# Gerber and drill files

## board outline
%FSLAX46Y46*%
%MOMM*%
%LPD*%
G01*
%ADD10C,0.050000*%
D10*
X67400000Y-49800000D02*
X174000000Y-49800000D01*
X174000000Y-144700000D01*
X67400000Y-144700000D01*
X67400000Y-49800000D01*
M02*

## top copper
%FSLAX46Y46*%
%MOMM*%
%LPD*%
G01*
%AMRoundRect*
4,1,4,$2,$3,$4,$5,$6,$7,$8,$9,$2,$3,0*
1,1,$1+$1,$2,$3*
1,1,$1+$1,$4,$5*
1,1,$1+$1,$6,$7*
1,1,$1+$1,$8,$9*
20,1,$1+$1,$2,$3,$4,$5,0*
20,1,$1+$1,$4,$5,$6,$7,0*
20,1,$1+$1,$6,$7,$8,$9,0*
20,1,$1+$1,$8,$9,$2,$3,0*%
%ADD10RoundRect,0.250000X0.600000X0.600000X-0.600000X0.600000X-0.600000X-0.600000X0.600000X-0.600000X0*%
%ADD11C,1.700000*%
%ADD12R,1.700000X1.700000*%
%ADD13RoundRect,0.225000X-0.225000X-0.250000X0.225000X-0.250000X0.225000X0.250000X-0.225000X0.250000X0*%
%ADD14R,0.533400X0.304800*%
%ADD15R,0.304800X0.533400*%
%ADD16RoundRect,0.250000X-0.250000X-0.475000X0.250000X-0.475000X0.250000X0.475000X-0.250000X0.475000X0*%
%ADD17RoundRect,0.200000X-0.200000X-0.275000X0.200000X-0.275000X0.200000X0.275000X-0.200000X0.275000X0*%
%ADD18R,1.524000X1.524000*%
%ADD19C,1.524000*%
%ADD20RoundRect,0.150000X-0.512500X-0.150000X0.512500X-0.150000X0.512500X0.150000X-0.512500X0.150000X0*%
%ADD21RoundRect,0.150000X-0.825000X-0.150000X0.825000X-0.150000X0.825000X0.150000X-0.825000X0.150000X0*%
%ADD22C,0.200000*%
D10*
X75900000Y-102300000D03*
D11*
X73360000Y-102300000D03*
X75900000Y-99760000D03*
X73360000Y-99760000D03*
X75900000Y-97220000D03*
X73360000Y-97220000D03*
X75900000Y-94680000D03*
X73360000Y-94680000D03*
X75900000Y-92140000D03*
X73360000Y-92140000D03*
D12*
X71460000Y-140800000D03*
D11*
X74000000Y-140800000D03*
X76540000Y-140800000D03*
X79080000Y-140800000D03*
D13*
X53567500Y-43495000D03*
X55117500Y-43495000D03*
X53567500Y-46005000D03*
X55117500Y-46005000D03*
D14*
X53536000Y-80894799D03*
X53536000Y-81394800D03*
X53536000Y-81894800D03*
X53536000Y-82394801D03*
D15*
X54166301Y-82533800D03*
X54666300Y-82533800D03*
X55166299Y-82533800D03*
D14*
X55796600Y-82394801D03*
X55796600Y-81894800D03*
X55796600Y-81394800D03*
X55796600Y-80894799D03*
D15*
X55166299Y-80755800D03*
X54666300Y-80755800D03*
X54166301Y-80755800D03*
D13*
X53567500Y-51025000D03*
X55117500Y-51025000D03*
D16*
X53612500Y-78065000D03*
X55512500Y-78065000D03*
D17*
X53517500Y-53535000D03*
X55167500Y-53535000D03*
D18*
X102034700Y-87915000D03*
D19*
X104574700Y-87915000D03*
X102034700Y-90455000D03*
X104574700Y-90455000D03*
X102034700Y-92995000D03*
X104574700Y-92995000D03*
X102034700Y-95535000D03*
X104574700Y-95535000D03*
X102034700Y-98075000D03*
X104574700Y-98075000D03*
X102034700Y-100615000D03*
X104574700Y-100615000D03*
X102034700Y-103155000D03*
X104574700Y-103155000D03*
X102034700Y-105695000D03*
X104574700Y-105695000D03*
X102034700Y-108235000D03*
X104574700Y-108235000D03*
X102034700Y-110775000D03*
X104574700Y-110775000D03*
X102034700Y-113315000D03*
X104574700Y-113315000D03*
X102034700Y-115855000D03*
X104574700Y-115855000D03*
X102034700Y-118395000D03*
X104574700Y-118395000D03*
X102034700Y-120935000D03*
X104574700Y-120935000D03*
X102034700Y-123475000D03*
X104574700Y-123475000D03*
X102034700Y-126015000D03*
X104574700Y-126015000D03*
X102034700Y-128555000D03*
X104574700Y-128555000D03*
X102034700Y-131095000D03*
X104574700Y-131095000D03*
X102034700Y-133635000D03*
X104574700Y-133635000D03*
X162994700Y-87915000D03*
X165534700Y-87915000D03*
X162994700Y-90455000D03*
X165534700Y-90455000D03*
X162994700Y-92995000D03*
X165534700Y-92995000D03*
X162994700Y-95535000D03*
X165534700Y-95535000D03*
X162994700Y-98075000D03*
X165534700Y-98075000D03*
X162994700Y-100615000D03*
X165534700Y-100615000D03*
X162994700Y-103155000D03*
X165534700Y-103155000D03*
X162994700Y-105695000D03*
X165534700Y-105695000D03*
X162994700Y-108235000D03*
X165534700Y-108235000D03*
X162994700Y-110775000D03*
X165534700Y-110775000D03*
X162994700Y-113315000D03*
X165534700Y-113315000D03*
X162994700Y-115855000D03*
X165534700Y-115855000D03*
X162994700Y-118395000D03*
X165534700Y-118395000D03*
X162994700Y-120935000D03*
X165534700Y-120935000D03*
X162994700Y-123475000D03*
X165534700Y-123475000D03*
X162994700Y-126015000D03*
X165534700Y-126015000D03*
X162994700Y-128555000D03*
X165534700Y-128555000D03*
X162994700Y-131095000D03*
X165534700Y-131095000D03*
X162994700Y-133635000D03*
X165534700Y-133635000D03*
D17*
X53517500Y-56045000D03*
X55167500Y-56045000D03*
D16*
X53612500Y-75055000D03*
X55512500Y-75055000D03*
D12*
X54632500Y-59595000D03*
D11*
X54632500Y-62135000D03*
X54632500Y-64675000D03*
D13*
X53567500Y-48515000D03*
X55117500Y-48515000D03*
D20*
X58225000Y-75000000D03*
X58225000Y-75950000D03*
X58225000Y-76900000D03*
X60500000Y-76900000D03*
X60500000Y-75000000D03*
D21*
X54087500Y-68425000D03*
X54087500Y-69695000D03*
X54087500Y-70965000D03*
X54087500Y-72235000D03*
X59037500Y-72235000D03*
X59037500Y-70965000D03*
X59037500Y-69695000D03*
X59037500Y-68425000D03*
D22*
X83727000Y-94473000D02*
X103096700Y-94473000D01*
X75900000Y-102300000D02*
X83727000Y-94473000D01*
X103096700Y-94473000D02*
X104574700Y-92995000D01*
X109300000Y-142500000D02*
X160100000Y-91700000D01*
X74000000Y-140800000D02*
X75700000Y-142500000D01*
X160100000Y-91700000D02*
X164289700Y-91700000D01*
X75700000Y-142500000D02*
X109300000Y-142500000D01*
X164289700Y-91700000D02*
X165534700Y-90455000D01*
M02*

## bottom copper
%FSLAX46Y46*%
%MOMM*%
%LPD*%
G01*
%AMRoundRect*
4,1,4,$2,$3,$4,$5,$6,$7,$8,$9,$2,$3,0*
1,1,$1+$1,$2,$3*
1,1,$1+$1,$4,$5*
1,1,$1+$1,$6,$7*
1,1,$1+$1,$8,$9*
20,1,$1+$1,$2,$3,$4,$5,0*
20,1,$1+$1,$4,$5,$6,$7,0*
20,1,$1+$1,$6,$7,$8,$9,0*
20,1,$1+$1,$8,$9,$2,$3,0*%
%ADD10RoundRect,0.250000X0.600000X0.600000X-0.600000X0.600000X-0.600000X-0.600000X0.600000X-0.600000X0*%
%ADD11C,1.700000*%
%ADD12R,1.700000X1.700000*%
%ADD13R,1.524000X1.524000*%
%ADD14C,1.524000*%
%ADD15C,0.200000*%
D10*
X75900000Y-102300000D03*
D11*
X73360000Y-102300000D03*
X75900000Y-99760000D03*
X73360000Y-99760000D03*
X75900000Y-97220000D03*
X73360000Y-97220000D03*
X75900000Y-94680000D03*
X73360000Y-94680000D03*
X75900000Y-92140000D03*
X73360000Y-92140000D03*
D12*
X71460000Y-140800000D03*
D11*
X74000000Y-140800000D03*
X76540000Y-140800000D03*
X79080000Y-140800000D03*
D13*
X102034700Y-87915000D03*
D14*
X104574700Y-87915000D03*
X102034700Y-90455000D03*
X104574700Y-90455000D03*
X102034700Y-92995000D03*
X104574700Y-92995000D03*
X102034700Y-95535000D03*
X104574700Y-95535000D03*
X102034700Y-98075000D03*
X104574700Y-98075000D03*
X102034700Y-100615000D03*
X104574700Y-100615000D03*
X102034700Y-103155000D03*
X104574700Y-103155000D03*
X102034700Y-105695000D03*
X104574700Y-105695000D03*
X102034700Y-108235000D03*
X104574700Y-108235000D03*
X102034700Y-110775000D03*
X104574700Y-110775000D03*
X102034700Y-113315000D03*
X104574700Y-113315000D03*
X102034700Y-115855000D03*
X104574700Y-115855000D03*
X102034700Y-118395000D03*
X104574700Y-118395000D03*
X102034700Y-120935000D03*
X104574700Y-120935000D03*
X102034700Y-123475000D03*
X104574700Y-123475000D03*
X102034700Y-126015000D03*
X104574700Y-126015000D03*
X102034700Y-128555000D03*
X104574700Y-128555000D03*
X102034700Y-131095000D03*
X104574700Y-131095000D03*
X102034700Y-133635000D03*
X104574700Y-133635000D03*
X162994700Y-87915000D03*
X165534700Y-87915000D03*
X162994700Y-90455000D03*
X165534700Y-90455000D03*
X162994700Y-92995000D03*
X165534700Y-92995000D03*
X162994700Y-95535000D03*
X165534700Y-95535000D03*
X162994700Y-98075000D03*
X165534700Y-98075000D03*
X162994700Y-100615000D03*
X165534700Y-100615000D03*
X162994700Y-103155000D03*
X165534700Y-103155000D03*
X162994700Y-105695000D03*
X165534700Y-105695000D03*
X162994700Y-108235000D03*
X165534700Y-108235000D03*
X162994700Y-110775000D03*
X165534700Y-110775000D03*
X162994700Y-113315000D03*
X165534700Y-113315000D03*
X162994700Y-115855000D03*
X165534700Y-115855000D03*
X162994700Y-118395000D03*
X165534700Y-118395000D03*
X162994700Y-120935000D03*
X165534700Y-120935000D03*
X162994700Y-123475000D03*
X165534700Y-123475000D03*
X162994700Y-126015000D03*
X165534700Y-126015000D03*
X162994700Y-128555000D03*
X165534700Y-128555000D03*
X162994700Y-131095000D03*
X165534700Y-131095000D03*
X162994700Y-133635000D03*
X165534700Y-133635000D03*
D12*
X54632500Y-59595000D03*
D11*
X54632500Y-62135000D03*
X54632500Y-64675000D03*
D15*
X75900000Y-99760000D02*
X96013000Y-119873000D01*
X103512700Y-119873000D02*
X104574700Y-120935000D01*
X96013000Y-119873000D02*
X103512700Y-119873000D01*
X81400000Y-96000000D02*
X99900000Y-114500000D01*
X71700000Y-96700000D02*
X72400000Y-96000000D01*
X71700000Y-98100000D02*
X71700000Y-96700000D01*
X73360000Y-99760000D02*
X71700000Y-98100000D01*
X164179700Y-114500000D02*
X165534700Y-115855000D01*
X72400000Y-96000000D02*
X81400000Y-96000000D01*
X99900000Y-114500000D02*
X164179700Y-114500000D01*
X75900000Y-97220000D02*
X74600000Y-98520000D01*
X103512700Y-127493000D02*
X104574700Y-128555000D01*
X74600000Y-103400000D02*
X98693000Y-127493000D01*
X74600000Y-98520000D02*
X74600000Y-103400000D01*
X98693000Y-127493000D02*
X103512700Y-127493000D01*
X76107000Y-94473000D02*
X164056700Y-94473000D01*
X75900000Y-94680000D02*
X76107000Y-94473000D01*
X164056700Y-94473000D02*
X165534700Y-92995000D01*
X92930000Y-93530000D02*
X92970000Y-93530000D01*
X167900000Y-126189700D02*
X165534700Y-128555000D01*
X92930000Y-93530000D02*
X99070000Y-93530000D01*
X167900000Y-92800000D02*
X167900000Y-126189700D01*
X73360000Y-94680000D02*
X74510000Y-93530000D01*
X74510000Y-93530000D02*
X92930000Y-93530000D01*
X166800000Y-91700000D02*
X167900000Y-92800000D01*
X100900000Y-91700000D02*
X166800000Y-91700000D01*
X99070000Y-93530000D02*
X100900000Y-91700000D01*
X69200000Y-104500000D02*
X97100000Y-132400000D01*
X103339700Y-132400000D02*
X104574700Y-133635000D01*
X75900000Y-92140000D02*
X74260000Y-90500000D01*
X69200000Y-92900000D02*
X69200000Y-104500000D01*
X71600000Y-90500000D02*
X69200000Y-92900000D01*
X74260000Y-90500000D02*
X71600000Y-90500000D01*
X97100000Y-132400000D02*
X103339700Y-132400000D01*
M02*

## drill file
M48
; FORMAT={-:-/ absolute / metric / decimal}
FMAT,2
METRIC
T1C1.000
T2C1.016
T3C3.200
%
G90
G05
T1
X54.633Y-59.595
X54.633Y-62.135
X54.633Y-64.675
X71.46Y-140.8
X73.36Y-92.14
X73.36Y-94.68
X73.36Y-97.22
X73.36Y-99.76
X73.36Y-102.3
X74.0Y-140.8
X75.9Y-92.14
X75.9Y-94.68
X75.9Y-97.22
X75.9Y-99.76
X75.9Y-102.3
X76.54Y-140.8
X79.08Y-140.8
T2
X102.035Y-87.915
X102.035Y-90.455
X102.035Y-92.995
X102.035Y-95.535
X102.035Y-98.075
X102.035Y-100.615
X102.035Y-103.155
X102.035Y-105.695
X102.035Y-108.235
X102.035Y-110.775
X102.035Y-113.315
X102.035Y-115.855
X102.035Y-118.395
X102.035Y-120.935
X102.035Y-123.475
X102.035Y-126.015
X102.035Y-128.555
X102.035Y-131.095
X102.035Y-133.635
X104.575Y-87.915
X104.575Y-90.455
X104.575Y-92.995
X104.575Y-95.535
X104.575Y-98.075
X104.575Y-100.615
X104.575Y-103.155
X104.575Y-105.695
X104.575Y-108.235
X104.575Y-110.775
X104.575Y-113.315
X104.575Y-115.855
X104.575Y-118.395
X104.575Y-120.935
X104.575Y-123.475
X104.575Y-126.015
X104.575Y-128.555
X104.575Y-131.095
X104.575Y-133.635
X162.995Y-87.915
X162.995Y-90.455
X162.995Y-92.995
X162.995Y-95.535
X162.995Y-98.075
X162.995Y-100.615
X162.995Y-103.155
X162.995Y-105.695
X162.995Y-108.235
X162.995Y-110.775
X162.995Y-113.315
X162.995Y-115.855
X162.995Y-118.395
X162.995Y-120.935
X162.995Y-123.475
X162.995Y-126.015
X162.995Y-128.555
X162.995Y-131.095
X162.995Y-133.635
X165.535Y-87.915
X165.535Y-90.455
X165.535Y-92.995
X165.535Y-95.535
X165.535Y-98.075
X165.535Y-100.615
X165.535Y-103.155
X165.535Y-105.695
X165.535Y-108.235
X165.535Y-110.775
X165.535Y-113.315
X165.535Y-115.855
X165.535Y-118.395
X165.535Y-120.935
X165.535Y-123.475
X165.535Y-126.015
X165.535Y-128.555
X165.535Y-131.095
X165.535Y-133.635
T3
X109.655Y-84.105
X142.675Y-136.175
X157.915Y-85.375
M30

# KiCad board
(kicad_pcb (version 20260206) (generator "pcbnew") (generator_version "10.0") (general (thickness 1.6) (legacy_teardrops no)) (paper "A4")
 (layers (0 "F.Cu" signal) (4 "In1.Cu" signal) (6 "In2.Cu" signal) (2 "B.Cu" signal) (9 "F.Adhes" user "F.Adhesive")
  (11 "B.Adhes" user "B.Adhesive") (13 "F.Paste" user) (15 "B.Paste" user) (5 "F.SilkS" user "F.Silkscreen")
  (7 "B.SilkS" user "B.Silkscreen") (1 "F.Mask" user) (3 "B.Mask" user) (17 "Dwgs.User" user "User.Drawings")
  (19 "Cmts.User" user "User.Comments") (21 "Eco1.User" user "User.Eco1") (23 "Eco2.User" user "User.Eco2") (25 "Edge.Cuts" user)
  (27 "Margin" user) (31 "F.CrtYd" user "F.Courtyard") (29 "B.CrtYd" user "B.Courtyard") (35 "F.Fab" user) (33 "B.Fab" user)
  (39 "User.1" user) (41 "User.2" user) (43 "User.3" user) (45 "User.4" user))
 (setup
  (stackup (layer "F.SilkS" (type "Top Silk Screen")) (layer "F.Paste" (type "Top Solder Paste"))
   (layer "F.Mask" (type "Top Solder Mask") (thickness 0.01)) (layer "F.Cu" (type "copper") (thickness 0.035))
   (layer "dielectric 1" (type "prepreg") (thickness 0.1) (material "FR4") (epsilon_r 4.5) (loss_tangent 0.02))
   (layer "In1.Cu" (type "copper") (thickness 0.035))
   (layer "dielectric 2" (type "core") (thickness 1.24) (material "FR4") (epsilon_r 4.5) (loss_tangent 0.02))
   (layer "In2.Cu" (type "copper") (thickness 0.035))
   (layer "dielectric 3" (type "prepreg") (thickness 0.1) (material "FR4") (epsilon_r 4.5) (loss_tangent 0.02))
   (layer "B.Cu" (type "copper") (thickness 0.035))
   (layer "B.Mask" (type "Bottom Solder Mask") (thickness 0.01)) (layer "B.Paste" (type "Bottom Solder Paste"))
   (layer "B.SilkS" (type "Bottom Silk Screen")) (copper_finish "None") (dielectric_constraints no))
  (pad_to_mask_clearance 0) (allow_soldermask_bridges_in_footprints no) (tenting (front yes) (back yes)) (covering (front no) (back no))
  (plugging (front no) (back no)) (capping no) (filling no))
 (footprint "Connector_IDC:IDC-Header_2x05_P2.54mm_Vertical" (layer "F.Cu") (at 75.9 102.3 180)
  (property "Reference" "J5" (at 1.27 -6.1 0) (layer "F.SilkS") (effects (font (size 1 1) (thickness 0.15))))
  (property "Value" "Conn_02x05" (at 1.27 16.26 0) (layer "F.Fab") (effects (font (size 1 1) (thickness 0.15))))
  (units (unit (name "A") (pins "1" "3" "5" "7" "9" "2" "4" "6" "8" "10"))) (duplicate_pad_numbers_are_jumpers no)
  (pad "1" thru_hole roundrect (at 0 0 180) (size 1.7 1.7) (drill 1) (layers "*.Cu" "*.Mask") (remove_unused_layers no)
   (roundrect_rratio 0.147059) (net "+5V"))
  (pad "2" thru_hole circle (at 2.54 0 180) (size 1.7 1.7) (drill 1) (layers "*.Cu" "*.Mask") (remove_unused_layers no) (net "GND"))
  (pad "3" thru_hole circle (at 0 2.54 180) (size 1.7 1.7) (drill 1) (layers "*.Cu" "*.Mask") (remove_unused_layers no) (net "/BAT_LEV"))
  (pad "4" thru_hole circle (at 2.54 2.54 180) (size 1.7 1.7) (drill 1) (layers "*.Cu" "*.Mask") (remove_unused_layers no) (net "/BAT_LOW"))
  (pad "5" thru_hole circle (at 0 5.08 180) (size 1.7 1.7) (drill 1) (layers "*.Cu" "*.Mask") (remove_unused_layers no) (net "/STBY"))
  (pad "6" thru_hole circle (at 2.54 5.08 180) (size 1.7 1.7) (drill 1) (layers "*.Cu" "*.Mask") (remove_unused_layers no) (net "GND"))
  (pad "7" thru_hole circle (at 0 7.62 180) (size 1.7 1.7) (drill 1) (layers "*.Cu" "*.Mask") (remove_unused_layers no) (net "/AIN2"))
  (pad "8" thru_hole circle (at 2.54 7.62 180) (size 1.7 1.7) (drill 1) (layers "*.Cu" "*.Mask") (remove_unused_layers no) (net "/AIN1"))
  (pad "9" thru_hole circle (at 0 10.16 180) (size 1.7 1.7) (drill 1) (layers "*.Cu" "*.Mask") (remove_unused_layers no) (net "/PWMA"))
  (pad "10" thru_hole circle (at 2.54 10.16 180) (size 1.7 1.7) (drill 1) (layers "*.Cu" "*.Mask") (remove_unused_layers no) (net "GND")))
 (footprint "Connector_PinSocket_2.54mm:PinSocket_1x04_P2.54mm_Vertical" (layer "F.Cu") (at 71.46 140.8 90)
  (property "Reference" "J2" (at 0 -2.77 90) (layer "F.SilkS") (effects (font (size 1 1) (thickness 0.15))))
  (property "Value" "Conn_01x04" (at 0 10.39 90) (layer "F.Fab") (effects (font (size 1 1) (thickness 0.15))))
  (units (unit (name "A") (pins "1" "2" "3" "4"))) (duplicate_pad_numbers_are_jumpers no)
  (pad "1" thru_hole rect (at 0 0 90) (size 1.7 1.7) (drill 1) (layers "*.Cu" "*.Mask") (remove_unused_layers no) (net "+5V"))
  (pad "2" thru_hole circle (at 0 2.54 90) (size 1.7 1.7) (drill 1) (layers "*.Cu" "*.Mask") (remove_unused_layers no) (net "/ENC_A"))
  (pad "3" thru_hole circle (at 0 5.08 90) (size 1.7 1.7) (drill 1) (layers "*.Cu" "*.Mask") (remove_unused_layers no) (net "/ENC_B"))
  (pad "4" thru_hole circle (at 0 7.62 90) (size 1.7 1.7) (drill 1) (layers "*.Cu" "*.Mask") (remove_unused_layers no) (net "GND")))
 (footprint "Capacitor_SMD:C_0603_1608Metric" (layer "F.Cu") (at 54.3425 43.495)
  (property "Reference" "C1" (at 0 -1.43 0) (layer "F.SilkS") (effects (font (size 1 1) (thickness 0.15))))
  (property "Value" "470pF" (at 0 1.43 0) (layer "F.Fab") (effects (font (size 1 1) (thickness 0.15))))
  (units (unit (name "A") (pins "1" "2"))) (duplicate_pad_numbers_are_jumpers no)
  (pad "1" smd roundrect (at -0.775 0) (size 0.9 0.95) (layers "F.Cu" "F.Mask" "F.Paste") (roundrect_rratio 0.25) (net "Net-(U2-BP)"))
  (pad "2" smd roundrect (at 0.775 0) (size 0.9 0.95) (layers "F.Cu" "F.Mask" "F.Paste") (roundrect_rratio 0.25) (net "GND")))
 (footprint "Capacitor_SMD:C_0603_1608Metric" (layer "F.Cu") (at 54.3425 46.005)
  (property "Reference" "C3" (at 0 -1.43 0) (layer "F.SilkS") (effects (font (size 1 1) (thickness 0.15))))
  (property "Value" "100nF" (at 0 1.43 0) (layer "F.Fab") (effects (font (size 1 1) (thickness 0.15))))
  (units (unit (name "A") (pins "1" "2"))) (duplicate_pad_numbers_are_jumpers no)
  (pad "1" smd roundrect (at -0.775 0) (size 0.9 0.95) (layers "F.Cu" "F.Mask" "F.Paste") (roundrect_rratio 0.25) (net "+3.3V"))
  (pad "2" smd roundrect (at 0.775 0) (size 0.9 0.95) (layers "F.Cu" "F.Mask" "F.Paste") (roundrect_rratio 0.25) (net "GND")))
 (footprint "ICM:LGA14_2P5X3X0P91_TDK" (layer "F.Cu") (at 54.6663 81.6448)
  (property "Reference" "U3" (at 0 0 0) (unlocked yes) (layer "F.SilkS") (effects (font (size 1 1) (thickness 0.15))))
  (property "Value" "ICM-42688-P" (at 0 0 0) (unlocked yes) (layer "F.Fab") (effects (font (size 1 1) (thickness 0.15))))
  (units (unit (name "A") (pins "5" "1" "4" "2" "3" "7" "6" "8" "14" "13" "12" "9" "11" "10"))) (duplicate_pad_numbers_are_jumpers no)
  (pad "1" smd rect (at -1.1303 -0.750001 90) (size 0.3048 0.5334) (layers "F.Cu" "F.Mask" "F.Paste") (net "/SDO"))
  (pad "2" smd rect (at -1.1303 -0.25 90) (size 0.3048 0.5334) (layers "F.Cu" "F.Mask" "F.Paste") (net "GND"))
  (pad "3" smd rect (at -1.1303 0.25 90) (size 0.3048 0.5334) (layers "F.Cu" "F.Mask" "F.Paste") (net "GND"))
  (pad "4" smd rect (at -1.1303 0.750001 90) (size 0.3048 0.5334) (layers "F.Cu" "F.Mask" "F.Paste") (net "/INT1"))
  (pad "5" smd rect (at -0.499999 0.889) (size 0.3048 0.5334) (layers "F.Cu" "F.Mask" "F.Paste") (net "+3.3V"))
  (pad "6" smd rect (at 0 0.889) (size 0.3048 0.5334) (layers "F.Cu" "F.Mask" "F.Paste") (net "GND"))
  (pad "7" smd rect (at 0.499999 0.889) (size 0.3048 0.5334) (layers "F.Cu" "F.Mask" "F.Paste") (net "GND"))
  (pad "8" smd rect (at 1.1303 0.750001 90) (size 0.3048 0.5334) (layers "F.Cu" "F.Mask" "F.Paste") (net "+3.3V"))
  (pad "9" smd rect (at 1.1303 0.25 90) (size 0.3048 0.5334) (layers "F.Cu" "F.Mask" "F.Paste") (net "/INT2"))
  (pad "10" smd rect (at 1.1303 -0.25 90) (size 0.3048 0.5334) (layers "F.Cu" "F.Mask" "F.Paste") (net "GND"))
  (pad "11" smd rect (at 1.1303 -0.750001 90) (size 0.3048 0.5334) (layers "F.Cu" "F.Mask" "F.Paste") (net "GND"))
  (pad "12" smd rect (at 0.499999 -0.889) (size 0.3048 0.5334) (layers "F.Cu" "F.Mask" "F.Paste") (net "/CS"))
  (pad "13" smd rect (at 0 -0.889) (size 0.3048 0.5334) (layers "F.Cu" "F.Mask" "F.Paste") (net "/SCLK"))
  (pad "14" smd rect (at -0.499999 -0.889) (size 0.3048 0.5334) (layers "F.Cu" "F.Mask" "F.Paste") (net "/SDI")))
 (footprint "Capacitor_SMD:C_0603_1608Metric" (layer "F.Cu") (at 54.3425 51.025)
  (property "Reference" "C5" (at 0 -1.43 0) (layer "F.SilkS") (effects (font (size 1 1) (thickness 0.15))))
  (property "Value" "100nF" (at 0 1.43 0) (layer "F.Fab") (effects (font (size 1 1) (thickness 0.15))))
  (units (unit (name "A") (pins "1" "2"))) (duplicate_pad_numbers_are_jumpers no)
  (pad "1" smd roundrect (at -0.775 0) (size 0.9 0.95) (layers "F.Cu" "F.Mask" "F.Paste") (roundrect_rratio 0.25) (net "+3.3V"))
  (pad "2" smd roundrect (at 0.775 0) (size 0.9 0.95) (layers "F.Cu" "F.Mask" "F.Paste") (roundrect_rratio 0.25) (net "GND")))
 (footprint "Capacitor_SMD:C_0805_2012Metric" (layer "F.Cu") (at 54.5625 78.065)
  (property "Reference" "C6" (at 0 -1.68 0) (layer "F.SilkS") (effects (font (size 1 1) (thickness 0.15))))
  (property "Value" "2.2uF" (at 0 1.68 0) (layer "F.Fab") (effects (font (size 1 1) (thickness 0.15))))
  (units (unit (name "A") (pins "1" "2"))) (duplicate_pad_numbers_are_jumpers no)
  (pad "1" smd roundrect (at -0.95 0) (size 1 1.45) (layers "F.Cu" "F.Mask" "F.Paste") (roundrect_rratio 0.25) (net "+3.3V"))
  (pad "2" smd roundrect (at 0.95 0) (size 1 1.45) (layers "F.Cu" "F.Mask" "F.Paste") (roundrect_rratio 0.25) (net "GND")))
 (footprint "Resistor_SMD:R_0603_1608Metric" (layer "F.Cu") (at 54.3425 53.535)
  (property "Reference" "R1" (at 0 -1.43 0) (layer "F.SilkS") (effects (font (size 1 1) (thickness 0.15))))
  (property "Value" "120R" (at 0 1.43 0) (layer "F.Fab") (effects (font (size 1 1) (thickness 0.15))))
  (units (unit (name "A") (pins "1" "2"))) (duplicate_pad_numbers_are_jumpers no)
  (pad "1" smd roundrect (at -0.825 0) (size 0.8 0.95) (layers "F.Cu" "F.Mask" "F.Paste") (roundrect_rratio 0.25) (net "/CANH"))
  (pad "2" smd roundrect (at 0.825 0) (size 0.8 0.95) (layers "F.Cu" "F.Mask" "F.Paste") (roundrect_rratio 0.25) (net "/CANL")))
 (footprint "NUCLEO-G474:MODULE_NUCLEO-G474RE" (layer "F.Cu") (at 133.7847 97.425)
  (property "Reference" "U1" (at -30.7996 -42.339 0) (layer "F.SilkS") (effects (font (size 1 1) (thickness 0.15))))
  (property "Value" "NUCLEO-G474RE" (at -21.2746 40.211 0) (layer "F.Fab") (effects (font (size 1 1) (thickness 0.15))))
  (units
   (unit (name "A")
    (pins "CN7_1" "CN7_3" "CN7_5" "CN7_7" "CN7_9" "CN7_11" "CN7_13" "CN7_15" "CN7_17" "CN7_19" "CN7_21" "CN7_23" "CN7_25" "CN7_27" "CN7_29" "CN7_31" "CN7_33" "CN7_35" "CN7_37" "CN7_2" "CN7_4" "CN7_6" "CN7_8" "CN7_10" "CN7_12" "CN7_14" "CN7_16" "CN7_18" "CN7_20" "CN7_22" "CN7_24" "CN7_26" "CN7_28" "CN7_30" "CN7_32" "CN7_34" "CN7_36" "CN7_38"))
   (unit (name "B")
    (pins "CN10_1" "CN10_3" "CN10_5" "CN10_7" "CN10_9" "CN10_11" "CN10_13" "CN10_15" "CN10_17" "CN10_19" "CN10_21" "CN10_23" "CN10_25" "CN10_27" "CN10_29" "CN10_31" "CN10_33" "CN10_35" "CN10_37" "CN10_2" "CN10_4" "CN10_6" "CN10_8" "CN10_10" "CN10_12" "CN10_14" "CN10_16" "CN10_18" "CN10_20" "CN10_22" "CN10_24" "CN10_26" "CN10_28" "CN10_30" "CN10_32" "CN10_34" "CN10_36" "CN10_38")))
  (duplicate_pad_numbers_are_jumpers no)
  (pad "" np_thru_hole circle (at -24.13 -13.32) (size 3.2 3.2) (drill 3.2) (layers "*.Cu" "*.Mask"))
  (pad "" np_thru_hole circle (at 8.89 38.75) (size 3.2 3.2) (drill 3.2) (layers "*.Cu" "*.Mask"))
  (pad "" np_thru_hole circle (at 24.13 -12.05) (size 3.2 3.2) (drill 3.2) (layers "*.Cu" "*.Mask"))
  (pad "CN7_1" thru_hole rect (at -31.75 -9.51) (size 1.524 1.524) (drill 1.016) (layers "*.Cu" "*.Mask") (remove_unused_layers no)
   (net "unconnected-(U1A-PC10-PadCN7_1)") (solder_mask_margin 0.102))
  (pad "CN7_2" thru_hole circle (at -29.21 -9.51) (size 1.524 1.524) (drill 1.016) (layers "*.Cu" "*.Mask") (remove_unused_layers no)
   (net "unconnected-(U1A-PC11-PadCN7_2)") (solder_mask_margin 0.102))
  (pad "CN7_3" thru_hole circle (at -31.75 -6.97) (size 1.524 1.524) (drill 1.016) (layers "*.Cu" "*.Mask") (remove_unused_layers no)
   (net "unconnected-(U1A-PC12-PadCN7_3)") (solder_mask_margin 0.102))
  (pad "CN7_4" thru_hole circle (at -29.21 -6.97) (size 1.524 1.524) (drill 1.016) (layers "*.Cu" "*.Mask") (remove_unused_layers no)
   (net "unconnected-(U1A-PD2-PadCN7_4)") (solder_mask_margin 0.102))
  (pad "CN7_5" thru_hole circle (at -31.75 -4.43) (size 1.524 1.524) (drill 1.016) (layers "*.Cu" "*.Mask") (remove_unused_layers no)
   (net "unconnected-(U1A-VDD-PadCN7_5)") (solder_mask_margin 0.102))
  (pad "CN7_6" thru_hole circle (at -29.21 -4.43) (size 1.524 1.524) (drill 1.016) (layers "*.Cu" "*.Mask") (remove_unused_layers no)
   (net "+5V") (solder_mask_margin 0.102))
  (pad "CN7_7" thru_hole circle (at -31.75 -1.89) (size 1.524 1.524) (drill 1.016) (layers "*.Cu" "*.Mask") (remove_unused_layers no)
   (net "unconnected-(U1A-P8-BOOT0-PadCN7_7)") (solder_mask_margin 0.102))
  (pad "CN7_8" thru_hole circle (at -29.21 -1.89) (size 1.524 1.524) (drill 1.016) (layers "*.Cu" "*.Mask") (remove_unused_layers no)
   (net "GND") (solder_mask_margin 0.102))
  (pad "CN7_9" thru_hole circle (at -31.75 0.65) (size 1.524 1.524) (drill 1.016) (layers "*.Cu" "*.Mask") (remove_unused_layers no)
   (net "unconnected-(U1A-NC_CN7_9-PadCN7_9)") (solder_mask_margin 0.102))
  (pad "CN7_10" thru_hole circle (at -29.21 0.65) (size 1.524 1.524) (drill 1.016) (layers "*.Cu" "*.Mask") (remove_unused_layers no)
   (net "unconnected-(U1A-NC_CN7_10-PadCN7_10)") (solder_mask_margin 0.102))
  (pad "CN7_11" thru_hole circle (at -31.75 3.19) (size 1.524 1.524) (drill 1.016) (layers "*.Cu" "*.Mask") (remove_unused_layers no)
   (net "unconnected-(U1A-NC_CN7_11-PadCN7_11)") (solder_mask_margin 0.102))
  (pad "CN7_12" thru_hole circle (at -29.21 3.19) (size 1.524 1.524) (drill 1.016) (layers "*.Cu" "*.Mask") (remove_unused_layers no)
   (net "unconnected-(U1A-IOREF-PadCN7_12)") (solder_mask_margin 0.102))
  (pad "CN7_13" thru_hole circle (at -31.75 5.73) (size 1.524 1.524) (drill 1.016) (layers "*.Cu" "*.Mask") (remove_unused_layers no)
   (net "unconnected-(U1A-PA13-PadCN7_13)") (solder_mask_margin 0.102))
  (pad "CN7_14" thru_hole circle (at -29.21 5.73) (size 1.524 1.524) (drill 1.016) (layers "*.Cu" "*.Mask") (remove_unused_layers no)
   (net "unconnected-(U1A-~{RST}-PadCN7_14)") (solder_mask_margin 0.102))
  (pad "CN7_15" thru_hole circle (at -31.75 8.27) (size 1.524 1.524) (drill 1.016) (layers "*.Cu" "*.Mask") (remove_unused_layers no)
   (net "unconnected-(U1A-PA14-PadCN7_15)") (solder_mask_margin 0.102))
  (pad "CN7_16" thru_hole circle (at -29.21 8.27) (size 1.524 1.524) (drill 1.016) (layers "*.Cu" "*.Mask") (remove_unused_layers no)
   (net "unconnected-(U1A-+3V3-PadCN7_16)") (solder_mask_margin 0.102))
  (pad "CN7_17" thru_hole circle (at -31.75 10.81) (size 1.524 1.524) (drill 1.016) (layers "*.Cu" "*.Mask") (remove_unused_layers no)
   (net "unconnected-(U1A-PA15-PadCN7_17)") (solder_mask_margin 0.102))
  (pad "CN7_18" thru_hole circle (at -29.21 10.81) (size 1.524 1.524) (drill 1.016) (layers "*.Cu" "*.Mask") (remove_unused_layers no)
   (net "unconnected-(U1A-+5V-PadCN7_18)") (solder_mask_margin 0.102))
  (pad "CN7_19" thru_hole circle (at -31.75 13.35) (size 1.524 1.524) (drill 1.016) (layers "*.Cu" "*.Mask") (remove_unused_layers no)
   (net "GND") (solder_mask_margin 0.102))
  (pad "CN7_20" thru_hole circle (at -29.21 13.35) (size 1.524 1.524) (drill 1.016) (layers "*.Cu" "*.Mask") (remove_unused_layers no)
   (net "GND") (solder_mask_margin 0.102))
  (pad "CN7_21" thru_hole circle (at -31.75 15.89) (size 1.524 1.524) (drill 1.016) (layers "*.Cu" "*.Mask") (remove_unused_layers no)
   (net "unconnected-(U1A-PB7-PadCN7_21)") (solder_mask_margin 0.102))
  (pad "CN7_22" thru_hole circle (at -29.21 15.89) (size 1.524 1.524) (drill 1.016) (layers "*.Cu" "*.Mask") (remove_unused_layers no)
   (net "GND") (solder_mask_margin 0.102))
  (pad "CN7_23" thru_hole circle (at -31.75 18.43) (size 1.524 1.524) (drill 1.016) (layers "*.Cu" "*.Mask") (remove_unused_layers no)
   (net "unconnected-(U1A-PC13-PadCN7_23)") (solder_mask_margin 0.102))
  (pad "CN7_24" thru_hole circle (at -29.21 18.43) (size 1.524 1.524) (drill 1.016) (layers "*.Cu" "*.Mask") (remove_unused_layers no)
   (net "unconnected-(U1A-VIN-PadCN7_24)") (solder_mask_margin 0.102))
  (pad "CN7_25" thru_hole circle (at -31.75 20.97) (size 1.524 1.524) (drill 1.016) (layers "*.Cu" "*.Mask") (remove_unused_layers no)
   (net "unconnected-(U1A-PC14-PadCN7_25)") (solder_mask_margin 0.102))
  (pad "CN7_26" thru_hole circle (at -29.21 20.97) (size 1.524 1.524) (drill 1.016) (layers "*.Cu" "*.Mask") (remove_unused_layers no)
   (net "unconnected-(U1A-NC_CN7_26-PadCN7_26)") (solder_mask_margin 0.102))
  (pad "CN7_27" thru_hole circle (at -31.75 23.51) (size 1.524 1.524) (drill 1.016) (layers "*.Cu" "*.Mask") (remove_unused_layers no)
   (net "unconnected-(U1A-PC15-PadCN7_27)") (solder_mask_margin 0.102))
  (pad "CN7_28" thru_hole circle (at -29.21 23.51) (size 1.524 1.524) (drill 1.016) (layers "*.Cu" "*.Mask") (remove_unused_layers no)
   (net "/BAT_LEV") (solder_mask_margin 0.102))
  (pad "CN7_29" thru_hole circle (at -31.75 26.05) (size 1.524 1.524) (drill 1.016) (layers "*.Cu" "*.Mask") (remove_unused_layers no)
   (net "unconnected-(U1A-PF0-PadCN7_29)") (solder_mask_margin 0.102))
  (pad "CN7_30" thru_hole circle (at -29.21 26.05) (size 1.524 1.524) (drill 1.016) (layers "*.Cu" "*.Mask") (remove_unused_layers no)
   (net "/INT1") (solder_mask_margin 0.102))
  (pad "CN7_31" thru_hole circle (at -31.75 28.59) (size 1.524 1.524) (drill 1.016) (layers "*.Cu" "*.Mask") (remove_unused_layers no)
   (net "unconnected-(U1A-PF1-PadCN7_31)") (solder_mask_margin 0.102))
  (pad "CN7_32" thru_hole circle (at -29.21 28.59) (size 1.524 1.524) (drill 1.016) (layers "*.Cu" "*.Mask") (remove_unused_layers no)
   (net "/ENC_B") (solder_mask_margin 0.102))
  (pad "CN7_33" thru_hole circle (at -31.75 31.13) (size 1.524 1.524) (drill 1.016) (layers "*.Cu" "*.Mask") (remove_unused_layers no)
   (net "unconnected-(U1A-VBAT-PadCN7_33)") (solder_mask_margin 0.102))
  (pad "CN7_34" thru_hole circle (at -29.21 31.13) (size 1.524 1.524) (drill 1.016) (layers "*.Cu" "*.Mask") (remove_unused_layers no)
   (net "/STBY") (solder_mask_margin 0.102))
  (pad "CN7_35" thru_hole circle (at -31.75 33.67) (size 1.524 1.524) (drill 1.016) (layers "*.Cu" "*.Mask") (remove_unused_layers no)
   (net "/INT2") (solder_mask_margin 0.102))
  (pad "CN7_36" thru_hole circle (at -29.21 33.67) (size 1.524 1.524) (drill 1.016) (layers "*.Cu" "*.Mask") (remove_unused_layers no)
   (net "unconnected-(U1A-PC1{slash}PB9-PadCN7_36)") (solder_mask_margin 0.102))
  (pad "CN7_37" thru_hole circle (at -31.75 36.21) (size 1.524 1.524) (drill 1.016) (layers "*.Cu" "*.Mask") (remove_unused_layers no)
   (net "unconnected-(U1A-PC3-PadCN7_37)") (solder_mask_margin 0.102))
  (pad "CN7_38" thru_hole circle (at -29.21 36.21) (size 1.524 1.524) (drill 1.016) (layers "*.Cu" "*.Mask") (remove_unused_layers no)
   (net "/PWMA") (solder_mask_margin 0.102))
  (pad "CN10_1" thru_hole circle (at 29.21 -9.51) (size 1.524 1.524) (drill 1.016) (layers "*.Cu" "*.Mask") (remove_unused_layers no)
   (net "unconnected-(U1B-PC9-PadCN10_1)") (solder_mask_margin 0.102))
  (pad "CN10_2" thru_hole circle (at 31.75 -9.51) (size 1.524 1.524) (drill 1.016) (layers "*.Cu" "*.Mask") (remove_unused_layers no)
   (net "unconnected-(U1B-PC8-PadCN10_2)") (solder_mask_margin 0.102))
  (pad "CN10_3" thru_hole circle (at 29.21 -6.97) (size 1.524 1.524) (drill 1.016) (layers "*.Cu" "*.Mask") (remove_unused_layers no)
   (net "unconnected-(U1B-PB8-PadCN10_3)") (solder_mask_margin 0.102))
  (pad "CN10_4" thru_hole circle (at 31.75 -6.97) (size 1.524 1.524) (drill 1.016) (layers "*.Cu" "*.Mask") (remove_unused_layers no)
   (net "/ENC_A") (solder_mask_margin 0.102))
  (pad "CN10_5" thru_hole circle (at 29.21 -4.43) (size 1.524 1.524) (drill 1.016) (layers "*.Cu" "*.Mask") (remove_unused_layers no)
   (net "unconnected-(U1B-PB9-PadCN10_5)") (solder_mask_margin 0.102))
  (pad "CN10_6" thru_hole circle (at 31.75 -4.43) (size 1.524 1.524) (drill 1.016) (layers "*.Cu" "*.Mask") (remove_unused_layers no)
   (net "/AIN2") (solder_mask_margin 0.102))
  (pad "CN10_7" thru_hole circle (at 29.21 -1.89) (size 1.524 1.524) (drill 1.016) (layers "*.Cu" "*.Mask") (remove_unused_layers no)
   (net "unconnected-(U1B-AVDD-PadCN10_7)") (solder_mask_margin 0.102))
  (pad "CN10_8" thru_hole circle (at 31.75 -1.89) (size 1.524 1.524) (drill 1.016) (layers "*.Cu" "*.Mask") (remove_unused_layers no)
   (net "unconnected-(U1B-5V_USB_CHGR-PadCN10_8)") (solder_mask_margin 0.102))
  (pad "CN10_9" thru_hole circle (at 29.21 0.65) (size 1.524 1.524) (drill 1.016) (layers "*.Cu" "*.Mask") (remove_unused_layers no)
   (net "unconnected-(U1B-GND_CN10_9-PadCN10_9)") (solder_mask_margin 0.102))
  (pad "CN10_10" thru_hole circle (at 31.75 0.65) (size 1.524 1.524) (drill 1.016) (layers "*.Cu" "*.Mask") (remove_unused_layers no)
   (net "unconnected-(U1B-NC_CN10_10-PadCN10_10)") (solder_mask_margin 0.102))
  (pad "CN10_11" thru_hole circle (at 29.21 3.19) (size 1.524 1.524) (drill 1.016) (layers "*.Cu" "*.Mask") (remove_unused_layers no)
   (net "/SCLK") (solder_mask_margin 0.102))
  (pad "CN10_12" thru_hole circle (at 31.75 3.19) (size 1.524 1.524) (drill 1.016) (layers "*.Cu" "*.Mask") (remove_unused_layers no)
   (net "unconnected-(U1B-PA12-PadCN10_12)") (solder_mask_margin 0.102))
  (pad "CN10_13" thru_hole circle (at 29.21 5.73) (size 1.524 1.524) (drill 1.016) (layers "*.Cu" "*.Mask") (remove_unused_layers no)
   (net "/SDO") (solder_mask_margin 0.102))
  (pad "CN10_14" thru_hole circle (at 31.75 5.73) (size 1.524 1.524) (drill 1.016) (layers "*.Cu" "*.Mask") (remove_unused_layers no)
   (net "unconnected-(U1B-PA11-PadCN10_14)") (solder_mask_margin 0.102))
  (pad "CN10_15" thru_hole circle (at 29.21 8.27) (size 1.524 1.524) (drill 1.016) (layers "*.Cu" "*.Mask") (remove_unused_layers no)
   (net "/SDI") (solder_mask_margin 0.102))
  (pad "CN10_16" thru_hole circle (at 31.75 8.27) (size 1.524 1.524) (drill 1.016) (layers "*.Cu" "*.Mask") (remove_unused_layers no)
   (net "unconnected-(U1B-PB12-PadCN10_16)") (solder_mask_margin 0.102))
  (pad "CN10_17" thru_hole circle (at 29.21 10.81) (size 1.524 1.524) (drill 1.016) (layers "*.Cu" "*.Mask") (remove_unused_layers no)
   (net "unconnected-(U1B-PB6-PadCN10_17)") (solder_mask_margin 0.102))
  (pad "CN10_18" thru_hole circle (at 31.75 10.81) (size 1.524 1.524) (drill 1.016) (layers "*.Cu" "*.Mask") (remove_unused_layers no)
   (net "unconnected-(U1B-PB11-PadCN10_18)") (solder_mask_margin 0.102))
  (pad "CN10_19" thru_hole circle (at 29.21 13.35) (size 1.524 1.524) (drill 1.016) (layers "*.Cu" "*.Mask") (remove_unused_layers no)
   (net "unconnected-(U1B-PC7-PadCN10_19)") (solder_mask_margin 0.102))
  (pad "CN10_20" thru_hole circle (at 31.75 13.35) (size 1.524 1.524) (drill 1.016) (layers "*.Cu" "*.Mask") (remove_unused_layers no)
   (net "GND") (solder_mask_margin 0.102))
  (pad "CN10_21" thru_hole circle (at 29.21 15.89) (size 1.524 1.524) (drill 1.016) (layers "*.Cu" "*.Mask") (remove_unused_layers no)
   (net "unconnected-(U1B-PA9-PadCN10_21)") (solder_mask_margin 0.102))
  (pad "CN10_22" thru_hole circle (at 31.75 15.89) (size 1.524 1.524) (drill 1.016) (layers "*.Cu" "*.Mask") (remove_unused_layers no)
   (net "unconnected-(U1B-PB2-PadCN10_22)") (solder_mask_margin 0.102))
  (pad "CN10_23" thru_hole circle (at 29.21 18.43) (size 1.524 1.524) (drill 1.016) (layers "*.Cu" "*.Mask") (remove_unused_layers no)
   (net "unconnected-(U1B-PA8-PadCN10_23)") (solder_mask_margin 0.102))
  (pad "CN10_24" thru_hole circle (at 31.75 18.43) (size 1.524 1.524) (drill 1.016) (layers "*.Cu" "*.Mask") (remove_unused_layers no)
   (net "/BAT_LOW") (solder_mask_margin 0.102))
  (pad "CN10_25" thru_hole circle (at 29.21 20.97) (size 1.524 1.524) (drill 1.016) (layers "*.Cu" "*.Mask") (remove_unused_layers no)
   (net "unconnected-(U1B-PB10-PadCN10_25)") (solder_mask_margin 0.102))
  (pad "CN10_26" thru_hole circle (at 31.75 20.97) (size 1.524 1.524) (drill 1.016) (layers "*.Cu" "*.Mask") (remove_unused_layers no)
   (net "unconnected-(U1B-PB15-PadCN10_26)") (solder_mask_margin 0.102))
  (pad "CN10_27" thru_hole circle (at 29.21 23.51) (size 1.524 1.524) (drill 1.016) (layers "*.Cu" "*.Mask") (remove_unused_layers no)
   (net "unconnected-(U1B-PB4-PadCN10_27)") (solder_mask_margin 0.102))
  (pad "CN10_28" thru_hole circle (at 31.75 23.51) (size 1.524 1.524) (drill 1.016) (layers "*.Cu" "*.Mask") (remove_unused_layers no)
   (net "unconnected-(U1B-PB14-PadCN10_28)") (solder_mask_margin 0.102))
  (pad "CN10_29" thru_hole circle (at 29.21 26.05) (size 1.524 1.524) (drill 1.016) (layers "*.Cu" "*.Mask") (remove_unused_layers no)
   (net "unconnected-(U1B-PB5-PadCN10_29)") (solder_mask_margin 0.102))
  (pad "CN10_30" thru_hole circle (at 31.75 26.05) (size 1.524 1.524) (drill 1.016) (layers "*.Cu" "*.Mask") (remove_unused_layers no)
   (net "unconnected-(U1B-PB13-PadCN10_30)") (solder_mask_margin 0.102))
  (pad "CN10_31" thru_hole circle (at 29.21 28.59) (size 1.524 1.524) (drill 1.016) (layers "*.Cu" "*.Mask") (remove_unused_layers no)
   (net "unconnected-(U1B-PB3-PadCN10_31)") (solder_mask_margin 0.102))
  (pad "CN10_32" thru_hole circle (at 31.75 28.59) (size 1.524 1.524) (drill 1.016) (layers "*.Cu" "*.Mask") (remove_unused_layers no)
   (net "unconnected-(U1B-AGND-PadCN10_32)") (solder_mask_margin 0.102))
  (pad "CN10_33" thru_hole circle (at 29.21 31.13) (size 1.524 1.524) (drill 1.016) (layers "*.Cu" "*.Mask") (remove_unused_layers no)
   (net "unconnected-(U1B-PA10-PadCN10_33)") (solder_mask_margin 0.102))
  (pad "CN10_34" thru_hole circle (at 31.75 31.13) (size 1.524 1.524) (drill 1.016) (layers "*.Cu" "*.Mask") (remove_unused_layers no)
   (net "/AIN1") (solder_mask_margin 0.102))
  (pad "CN10_35" thru_hole circle (at 29.21 33.67) (size 1.524 1.524) (drill 1.016) (layers "*.Cu" "*.Mask") (remove_unused_layers no)
   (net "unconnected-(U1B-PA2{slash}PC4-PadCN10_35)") (solder_mask_margin 0.102))
  (pad "CN10_36" thru_hole circle (at 31.75 33.67) (size 1.524 1.524) (drill 1.016) (layers "*.Cu" "*.Mask") (remove_unused_layers no)
   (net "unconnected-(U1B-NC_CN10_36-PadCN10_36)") (solder_mask_margin 0.102))
  (pad "CN10_37" thru_hole circle (at 29.21 36.21) (size 1.524 1.524) (drill 1.016) (layers "*.Cu" "*.Mask") (remove_unused_layers no)
   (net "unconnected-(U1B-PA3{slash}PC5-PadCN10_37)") (solder_mask_margin 0.102))
  (pad "CN10_38" thru_hole circle (at 31.75 36.21) (size 1.524 1.524) (drill 1.016) (layers "*.Cu" "*.Mask") (remove_unused_layers no)
   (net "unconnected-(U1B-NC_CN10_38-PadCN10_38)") (solder_mask_margin 0.102)))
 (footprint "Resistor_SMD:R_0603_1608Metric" (layer "F.Cu") (at 54.3425 56.045)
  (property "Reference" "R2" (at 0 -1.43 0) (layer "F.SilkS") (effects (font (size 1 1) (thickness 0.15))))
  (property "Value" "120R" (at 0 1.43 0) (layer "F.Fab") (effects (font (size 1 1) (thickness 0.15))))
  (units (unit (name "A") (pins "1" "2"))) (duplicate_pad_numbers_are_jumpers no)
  (pad "1" smd roundrect (at -0.825 0) (size 0.8 0.95) (layers "F.Cu" "F.Mask" "F.Paste") (roundrect_rratio 0.25) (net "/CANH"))
  (pad "2" smd roundrect (at 0.825 0) (size 0.8 0.95) (layers "F.Cu" "F.Mask" "F.Paste") (roundrect_rratio 0.25) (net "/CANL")))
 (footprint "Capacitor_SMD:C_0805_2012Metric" (layer "F.Cu") (at 54.5625 75.055)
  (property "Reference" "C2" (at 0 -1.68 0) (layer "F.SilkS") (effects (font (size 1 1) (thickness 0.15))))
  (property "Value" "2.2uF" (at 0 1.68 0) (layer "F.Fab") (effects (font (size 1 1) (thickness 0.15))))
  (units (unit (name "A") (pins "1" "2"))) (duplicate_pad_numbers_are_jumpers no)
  (pad "1" smd roundrect (at -0.95 0) (size 1 1.45) (layers "F.Cu" "F.Mask" "F.Paste") (roundrect_rratio 0.25) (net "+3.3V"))
  (pad "2" smd roundrect (at 0.95 0) (size 1 1.45) (layers "F.Cu" "F.Mask" "F.Paste") (roundrect_rratio 0.25) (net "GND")))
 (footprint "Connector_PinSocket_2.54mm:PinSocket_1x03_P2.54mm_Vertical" (layer "F.Cu") (at 54.6325 59.595)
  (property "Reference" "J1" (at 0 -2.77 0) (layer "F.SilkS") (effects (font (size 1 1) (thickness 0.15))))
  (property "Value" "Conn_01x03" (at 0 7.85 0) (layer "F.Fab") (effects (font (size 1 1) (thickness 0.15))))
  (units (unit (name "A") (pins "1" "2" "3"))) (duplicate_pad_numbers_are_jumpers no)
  (pad "1" thru_hole rect (at 0 0) (size 1.7 1.7) (drill 1) (layers "*.Cu" "*.Mask") (remove_unused_layers no) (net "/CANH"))
  (pad "2" thru_hole circle (at 0 2.54) (size 1.7 1.7) (drill 1) (layers "*.Cu" "*.Mask") (remove_unused_layers no) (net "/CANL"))
  (pad "3" thru_hole circle (at 0 5.08) (size 1.7 1.7) (drill 1) (layers "*.Cu" "*.Mask") (remove_unused_layers no) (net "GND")))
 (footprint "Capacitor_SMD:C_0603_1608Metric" (layer "F.Cu") (at 54.3425 48.515)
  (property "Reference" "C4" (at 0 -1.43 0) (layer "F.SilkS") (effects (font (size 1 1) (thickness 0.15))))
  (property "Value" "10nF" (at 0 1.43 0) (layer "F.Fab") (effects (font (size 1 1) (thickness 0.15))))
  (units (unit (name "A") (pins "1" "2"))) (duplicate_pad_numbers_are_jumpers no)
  (pad "1" smd roundrect (at -0.775 0) (size 0.9 0.95) (layers "F.Cu" "F.Mask" "F.Paste") (roundrect_rratio 0.25) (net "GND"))
  (pad "2" smd roundrect (at 0.775 0) (size 0.9 0.95) (layers "F.Cu" "F.Mask" "F.Paste") (roundrect_rratio 0.25) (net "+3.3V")))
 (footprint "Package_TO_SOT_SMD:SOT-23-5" (layer "F.Cu") (at 59.3625 75.95)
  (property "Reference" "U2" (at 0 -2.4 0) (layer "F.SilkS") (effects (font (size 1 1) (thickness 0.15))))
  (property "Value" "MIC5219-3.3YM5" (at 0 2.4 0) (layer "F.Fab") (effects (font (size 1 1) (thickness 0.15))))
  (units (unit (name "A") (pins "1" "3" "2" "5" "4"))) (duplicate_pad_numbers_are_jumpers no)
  (pad "1" smd roundrect (at -1.1375 -0.95) (size 1.325 0.6) (layers "F.Cu" "F.Mask" "F.Paste") (roundrect_rratio 0.25) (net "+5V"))
  (pad "2" smd roundrect (at -1.1375 0) (size 1.325 0.6) (layers "F.Cu" "F.Mask" "F.Paste") (roundrect_rratio 0.25) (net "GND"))
  (pad "3" smd roundrect (at -1.1375 0.95) (size 1.325 0.6) (layers "F.Cu" "F.Mask" "F.Paste") (roundrect_rratio 0.25) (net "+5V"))
  (pad "4" smd roundrect (at 1.1375 0.95) (size 1.325 0.6) (layers "F.Cu" "F.Mask" "F.Paste") (roundrect_rratio 0.25) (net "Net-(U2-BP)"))
  (pad "5" smd roundrect (at 1.1375 -0.95) (size 1.325 0.6) (layers "F.Cu" "F.Mask" "F.Paste") (roundrect_rratio 0.25) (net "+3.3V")))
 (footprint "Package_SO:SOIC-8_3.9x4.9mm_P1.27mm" (layer "F.Cu") (at 56.5625 70.33)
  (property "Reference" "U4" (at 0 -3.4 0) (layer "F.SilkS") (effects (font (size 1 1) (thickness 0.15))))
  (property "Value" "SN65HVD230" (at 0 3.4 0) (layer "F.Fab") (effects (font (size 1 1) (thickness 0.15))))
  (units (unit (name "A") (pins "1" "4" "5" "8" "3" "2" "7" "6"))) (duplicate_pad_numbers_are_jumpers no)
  (pad "1" smd roundrect (at -2.475 -1.905) (size 1.95 0.6) (layers "F.Cu" "F.Mask" "F.Paste") (roundrect_rratio 0.25) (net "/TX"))
  (pad "2" smd roundrect (at -2.475 -0.635) (size 1.95 0.6) (layers "F.Cu" "F.Mask" "F.Paste") (roundrect_rratio 0.25) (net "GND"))
  (pad "3" smd roundrect (at -2.475 0.635) (size 1.95 0.6) (layers "F.Cu" "F.Mask" "F.Paste") (roundrect_rratio 0.25) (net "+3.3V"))
  (pad "4" smd roundrect (at -2.475 1.905) (size 1.95 0.6) (layers "F.Cu" "F.Mask" "F.Paste") (roundrect_rratio 0.25) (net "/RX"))
  (pad "5" smd roundrect (at 2.475 1.905) (size 1.95 0.6) (layers "F.Cu" "F.Mask" "F.Paste") (roundrect_rratio 0.25)
   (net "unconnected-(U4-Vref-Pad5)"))
  (pad "6" smd roundrect (at 2.475 0.635) (size 1.95 0.6) (layers "F.Cu" "F.Mask" "F.Paste") (roundrect_rratio 0.25) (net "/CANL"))
  (pad "7" smd roundrect (at 2.475 -0.635) (size 1.95 0.6) (layers "F.Cu" "F.Mask" "F.Paste") (roundrect_rratio 0.25) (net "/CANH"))
  (pad "8" smd roundrect (at 2.475 -1.905) (size 1.95 0.6) (layers "F.Cu" "F.Mask" "F.Paste") (roundrect_rratio 0.25) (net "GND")))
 (gr_rect (start 67.4 49.8) (end 174 144.7) (stroke (width 0.05) (type default)) (fill no) (layer "Edge.Cuts"))
 (segment (start 83.727 94.473) (end 103.0967 94.473) (width 0.2) (layer "F.Cu") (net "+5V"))
 (segment (start 75.9 102.3) (end 83.727 94.473) (width 0.2) (layer "F.Cu") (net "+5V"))
 (segment (start 103.0967 94.473) (end 104.5747 92.995) (width 0.2) (layer "F.Cu") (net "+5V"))
 (segment (start 75.9 99.76) (end 96.013 119.873) (width 0.2) (layer "B.Cu") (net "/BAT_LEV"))
 (segment (start 103.5127 119.873) (end 104.5747 120.935) (width 0.2) (layer "B.Cu") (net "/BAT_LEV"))
 (segment (start 96.013 119.873) (end 103.5127 119.873) (width 0.2) (layer "B.Cu") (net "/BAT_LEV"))
 (segment (start 81.4 96) (end 99.9 114.5) (width 0.2) (layer "B.Cu") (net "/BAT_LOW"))
 (segment (start 71.7 96.7) (end 72.4 96) (width 0.2) (layer "B.Cu") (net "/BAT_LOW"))
 (segment (start 71.7 98.1) (end 71.7 96.7) (width 0.2) (layer "B.Cu") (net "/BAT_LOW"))
 (segment (start 73.36 99.76) (end 71.7 98.1) (width 0.2) (layer "B.Cu") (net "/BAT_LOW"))
 (segment (start 164.1797 114.5) (end 165.5347 115.855) (width 0.2) (layer "B.Cu") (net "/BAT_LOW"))
 (segment (start 72.4 96) (end 81.4 96) (width 0.2) (layer "B.Cu") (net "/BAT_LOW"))
 (segment (start 99.9 114.5) (end 164.1797 114.5) (width 0.2) (layer "B.Cu") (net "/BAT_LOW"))
 (segment (start 75.9 97.22) (end 74.6 98.52) (width 0.2) (layer "B.Cu") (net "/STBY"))
 (segment (start 103.5127 127.493) (end 104.5747 128.555) (width 0.2) (layer "B.Cu") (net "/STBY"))
 (segment (start 74.6 103.4) (end 98.693 127.493) (width 0.2) (layer "B.Cu") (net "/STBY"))
 (segment (start 74.6 98.52) (end 74.6 103.4) (width 0.2) (layer "B.Cu") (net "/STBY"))
 (segment (start 98.693 127.493) (end 103.5127 127.493) (width 0.2) (layer "B.Cu") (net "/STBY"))
 (segment (start 76.107 94.473) (end 164.0567 94.473) (width 0.2) (layer "B.Cu") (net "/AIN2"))
 (segment (start 75.9 94.68) (end 76.107 94.473) (width 0.2) (layer "B.Cu") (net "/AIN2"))
 (segment (start 164.0567 94.473) (end 165.5347 92.995) (width 0.2) (layer "B.Cu") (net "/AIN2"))
 (segment (start 92.93 93.53) (end 92.97 93.53) (width 0.2) (layer "B.Cu") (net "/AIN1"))
 (segment (start 167.9 126.1897) (end 165.5347 128.555) (width 0.2) (layer "B.Cu") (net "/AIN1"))
 (segment (start 92.93 93.53) (end 99.07 93.53) (width 0.2) (layer "B.Cu") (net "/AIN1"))
 (segment (start 167.9 92.8) (end 167.9 126.1897) (width 0.2) (layer "B.Cu") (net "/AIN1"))
 (segment (start 73.36 94.68) (end 74.51 93.53) (width 0.2) (layer "B.Cu") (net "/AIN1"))
 (segment (start 74.51 93.53) (end 92.93 93.53) (width 0.2) (layer "B.Cu") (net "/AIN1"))
 (segment (start 166.8 91.7) (end 167.9 92.8) (width 0.2) (layer "B.Cu") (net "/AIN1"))
 (segment (start 100.9 91.7) (end 166.8 91.7) (width 0.2) (layer "B.Cu") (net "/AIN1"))
 (segment (start 99.07 93.53) (end 100.9 91.7) (width 0.2) (layer "B.Cu") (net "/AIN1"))
 (segment (start 69.2 104.5) (end 97.1 132.4) (width 0.2) (layer "B.Cu") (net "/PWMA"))
 (segment (start 103.3397 132.4) (end 104.5747 133.635) (width 0.2) (layer "B.Cu") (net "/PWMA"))
 (segment (start 75.9 92.14) (end 74.26 90.5) (width 0.2) (layer "B.Cu") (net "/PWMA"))
 (segment (start 69.2 92.9) (end 69.2 104.5) (width 0.2) (layer "B.Cu") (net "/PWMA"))
 (segment (start 71.6 90.5) (end 69.2 92.9) (width 0.2) (layer "B.Cu") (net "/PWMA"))
 (segment (start 74.26 90.5) (end 71.6 90.5) (width 0.2) (layer "B.Cu") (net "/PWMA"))
 (segment (start 97.1 132.4) (end 103.3397 132.4) (width 0.2) (layer "B.Cu") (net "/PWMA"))
 (segment (start 109.3 142.5) (end 160.1 91.7) (width 0.2) (layer "F.Cu") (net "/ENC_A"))
 (segment (start 74 140.8) (end 75.7 142.5) (width 0.2) (layer "F.Cu") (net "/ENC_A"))
 (segment (start 160.1 91.7) (end 164.2897 91.7) (width 0.2) (layer "F.Cu") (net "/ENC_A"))
 (segment (start 75.7 142.5) (end 109.3 142.5) (width 0.2) (layer "F.Cu") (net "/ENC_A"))
 (segment (start 164.2897 91.7) (end 165.5347 90.455) (width 0.2) (layer "F.Cu") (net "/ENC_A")))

